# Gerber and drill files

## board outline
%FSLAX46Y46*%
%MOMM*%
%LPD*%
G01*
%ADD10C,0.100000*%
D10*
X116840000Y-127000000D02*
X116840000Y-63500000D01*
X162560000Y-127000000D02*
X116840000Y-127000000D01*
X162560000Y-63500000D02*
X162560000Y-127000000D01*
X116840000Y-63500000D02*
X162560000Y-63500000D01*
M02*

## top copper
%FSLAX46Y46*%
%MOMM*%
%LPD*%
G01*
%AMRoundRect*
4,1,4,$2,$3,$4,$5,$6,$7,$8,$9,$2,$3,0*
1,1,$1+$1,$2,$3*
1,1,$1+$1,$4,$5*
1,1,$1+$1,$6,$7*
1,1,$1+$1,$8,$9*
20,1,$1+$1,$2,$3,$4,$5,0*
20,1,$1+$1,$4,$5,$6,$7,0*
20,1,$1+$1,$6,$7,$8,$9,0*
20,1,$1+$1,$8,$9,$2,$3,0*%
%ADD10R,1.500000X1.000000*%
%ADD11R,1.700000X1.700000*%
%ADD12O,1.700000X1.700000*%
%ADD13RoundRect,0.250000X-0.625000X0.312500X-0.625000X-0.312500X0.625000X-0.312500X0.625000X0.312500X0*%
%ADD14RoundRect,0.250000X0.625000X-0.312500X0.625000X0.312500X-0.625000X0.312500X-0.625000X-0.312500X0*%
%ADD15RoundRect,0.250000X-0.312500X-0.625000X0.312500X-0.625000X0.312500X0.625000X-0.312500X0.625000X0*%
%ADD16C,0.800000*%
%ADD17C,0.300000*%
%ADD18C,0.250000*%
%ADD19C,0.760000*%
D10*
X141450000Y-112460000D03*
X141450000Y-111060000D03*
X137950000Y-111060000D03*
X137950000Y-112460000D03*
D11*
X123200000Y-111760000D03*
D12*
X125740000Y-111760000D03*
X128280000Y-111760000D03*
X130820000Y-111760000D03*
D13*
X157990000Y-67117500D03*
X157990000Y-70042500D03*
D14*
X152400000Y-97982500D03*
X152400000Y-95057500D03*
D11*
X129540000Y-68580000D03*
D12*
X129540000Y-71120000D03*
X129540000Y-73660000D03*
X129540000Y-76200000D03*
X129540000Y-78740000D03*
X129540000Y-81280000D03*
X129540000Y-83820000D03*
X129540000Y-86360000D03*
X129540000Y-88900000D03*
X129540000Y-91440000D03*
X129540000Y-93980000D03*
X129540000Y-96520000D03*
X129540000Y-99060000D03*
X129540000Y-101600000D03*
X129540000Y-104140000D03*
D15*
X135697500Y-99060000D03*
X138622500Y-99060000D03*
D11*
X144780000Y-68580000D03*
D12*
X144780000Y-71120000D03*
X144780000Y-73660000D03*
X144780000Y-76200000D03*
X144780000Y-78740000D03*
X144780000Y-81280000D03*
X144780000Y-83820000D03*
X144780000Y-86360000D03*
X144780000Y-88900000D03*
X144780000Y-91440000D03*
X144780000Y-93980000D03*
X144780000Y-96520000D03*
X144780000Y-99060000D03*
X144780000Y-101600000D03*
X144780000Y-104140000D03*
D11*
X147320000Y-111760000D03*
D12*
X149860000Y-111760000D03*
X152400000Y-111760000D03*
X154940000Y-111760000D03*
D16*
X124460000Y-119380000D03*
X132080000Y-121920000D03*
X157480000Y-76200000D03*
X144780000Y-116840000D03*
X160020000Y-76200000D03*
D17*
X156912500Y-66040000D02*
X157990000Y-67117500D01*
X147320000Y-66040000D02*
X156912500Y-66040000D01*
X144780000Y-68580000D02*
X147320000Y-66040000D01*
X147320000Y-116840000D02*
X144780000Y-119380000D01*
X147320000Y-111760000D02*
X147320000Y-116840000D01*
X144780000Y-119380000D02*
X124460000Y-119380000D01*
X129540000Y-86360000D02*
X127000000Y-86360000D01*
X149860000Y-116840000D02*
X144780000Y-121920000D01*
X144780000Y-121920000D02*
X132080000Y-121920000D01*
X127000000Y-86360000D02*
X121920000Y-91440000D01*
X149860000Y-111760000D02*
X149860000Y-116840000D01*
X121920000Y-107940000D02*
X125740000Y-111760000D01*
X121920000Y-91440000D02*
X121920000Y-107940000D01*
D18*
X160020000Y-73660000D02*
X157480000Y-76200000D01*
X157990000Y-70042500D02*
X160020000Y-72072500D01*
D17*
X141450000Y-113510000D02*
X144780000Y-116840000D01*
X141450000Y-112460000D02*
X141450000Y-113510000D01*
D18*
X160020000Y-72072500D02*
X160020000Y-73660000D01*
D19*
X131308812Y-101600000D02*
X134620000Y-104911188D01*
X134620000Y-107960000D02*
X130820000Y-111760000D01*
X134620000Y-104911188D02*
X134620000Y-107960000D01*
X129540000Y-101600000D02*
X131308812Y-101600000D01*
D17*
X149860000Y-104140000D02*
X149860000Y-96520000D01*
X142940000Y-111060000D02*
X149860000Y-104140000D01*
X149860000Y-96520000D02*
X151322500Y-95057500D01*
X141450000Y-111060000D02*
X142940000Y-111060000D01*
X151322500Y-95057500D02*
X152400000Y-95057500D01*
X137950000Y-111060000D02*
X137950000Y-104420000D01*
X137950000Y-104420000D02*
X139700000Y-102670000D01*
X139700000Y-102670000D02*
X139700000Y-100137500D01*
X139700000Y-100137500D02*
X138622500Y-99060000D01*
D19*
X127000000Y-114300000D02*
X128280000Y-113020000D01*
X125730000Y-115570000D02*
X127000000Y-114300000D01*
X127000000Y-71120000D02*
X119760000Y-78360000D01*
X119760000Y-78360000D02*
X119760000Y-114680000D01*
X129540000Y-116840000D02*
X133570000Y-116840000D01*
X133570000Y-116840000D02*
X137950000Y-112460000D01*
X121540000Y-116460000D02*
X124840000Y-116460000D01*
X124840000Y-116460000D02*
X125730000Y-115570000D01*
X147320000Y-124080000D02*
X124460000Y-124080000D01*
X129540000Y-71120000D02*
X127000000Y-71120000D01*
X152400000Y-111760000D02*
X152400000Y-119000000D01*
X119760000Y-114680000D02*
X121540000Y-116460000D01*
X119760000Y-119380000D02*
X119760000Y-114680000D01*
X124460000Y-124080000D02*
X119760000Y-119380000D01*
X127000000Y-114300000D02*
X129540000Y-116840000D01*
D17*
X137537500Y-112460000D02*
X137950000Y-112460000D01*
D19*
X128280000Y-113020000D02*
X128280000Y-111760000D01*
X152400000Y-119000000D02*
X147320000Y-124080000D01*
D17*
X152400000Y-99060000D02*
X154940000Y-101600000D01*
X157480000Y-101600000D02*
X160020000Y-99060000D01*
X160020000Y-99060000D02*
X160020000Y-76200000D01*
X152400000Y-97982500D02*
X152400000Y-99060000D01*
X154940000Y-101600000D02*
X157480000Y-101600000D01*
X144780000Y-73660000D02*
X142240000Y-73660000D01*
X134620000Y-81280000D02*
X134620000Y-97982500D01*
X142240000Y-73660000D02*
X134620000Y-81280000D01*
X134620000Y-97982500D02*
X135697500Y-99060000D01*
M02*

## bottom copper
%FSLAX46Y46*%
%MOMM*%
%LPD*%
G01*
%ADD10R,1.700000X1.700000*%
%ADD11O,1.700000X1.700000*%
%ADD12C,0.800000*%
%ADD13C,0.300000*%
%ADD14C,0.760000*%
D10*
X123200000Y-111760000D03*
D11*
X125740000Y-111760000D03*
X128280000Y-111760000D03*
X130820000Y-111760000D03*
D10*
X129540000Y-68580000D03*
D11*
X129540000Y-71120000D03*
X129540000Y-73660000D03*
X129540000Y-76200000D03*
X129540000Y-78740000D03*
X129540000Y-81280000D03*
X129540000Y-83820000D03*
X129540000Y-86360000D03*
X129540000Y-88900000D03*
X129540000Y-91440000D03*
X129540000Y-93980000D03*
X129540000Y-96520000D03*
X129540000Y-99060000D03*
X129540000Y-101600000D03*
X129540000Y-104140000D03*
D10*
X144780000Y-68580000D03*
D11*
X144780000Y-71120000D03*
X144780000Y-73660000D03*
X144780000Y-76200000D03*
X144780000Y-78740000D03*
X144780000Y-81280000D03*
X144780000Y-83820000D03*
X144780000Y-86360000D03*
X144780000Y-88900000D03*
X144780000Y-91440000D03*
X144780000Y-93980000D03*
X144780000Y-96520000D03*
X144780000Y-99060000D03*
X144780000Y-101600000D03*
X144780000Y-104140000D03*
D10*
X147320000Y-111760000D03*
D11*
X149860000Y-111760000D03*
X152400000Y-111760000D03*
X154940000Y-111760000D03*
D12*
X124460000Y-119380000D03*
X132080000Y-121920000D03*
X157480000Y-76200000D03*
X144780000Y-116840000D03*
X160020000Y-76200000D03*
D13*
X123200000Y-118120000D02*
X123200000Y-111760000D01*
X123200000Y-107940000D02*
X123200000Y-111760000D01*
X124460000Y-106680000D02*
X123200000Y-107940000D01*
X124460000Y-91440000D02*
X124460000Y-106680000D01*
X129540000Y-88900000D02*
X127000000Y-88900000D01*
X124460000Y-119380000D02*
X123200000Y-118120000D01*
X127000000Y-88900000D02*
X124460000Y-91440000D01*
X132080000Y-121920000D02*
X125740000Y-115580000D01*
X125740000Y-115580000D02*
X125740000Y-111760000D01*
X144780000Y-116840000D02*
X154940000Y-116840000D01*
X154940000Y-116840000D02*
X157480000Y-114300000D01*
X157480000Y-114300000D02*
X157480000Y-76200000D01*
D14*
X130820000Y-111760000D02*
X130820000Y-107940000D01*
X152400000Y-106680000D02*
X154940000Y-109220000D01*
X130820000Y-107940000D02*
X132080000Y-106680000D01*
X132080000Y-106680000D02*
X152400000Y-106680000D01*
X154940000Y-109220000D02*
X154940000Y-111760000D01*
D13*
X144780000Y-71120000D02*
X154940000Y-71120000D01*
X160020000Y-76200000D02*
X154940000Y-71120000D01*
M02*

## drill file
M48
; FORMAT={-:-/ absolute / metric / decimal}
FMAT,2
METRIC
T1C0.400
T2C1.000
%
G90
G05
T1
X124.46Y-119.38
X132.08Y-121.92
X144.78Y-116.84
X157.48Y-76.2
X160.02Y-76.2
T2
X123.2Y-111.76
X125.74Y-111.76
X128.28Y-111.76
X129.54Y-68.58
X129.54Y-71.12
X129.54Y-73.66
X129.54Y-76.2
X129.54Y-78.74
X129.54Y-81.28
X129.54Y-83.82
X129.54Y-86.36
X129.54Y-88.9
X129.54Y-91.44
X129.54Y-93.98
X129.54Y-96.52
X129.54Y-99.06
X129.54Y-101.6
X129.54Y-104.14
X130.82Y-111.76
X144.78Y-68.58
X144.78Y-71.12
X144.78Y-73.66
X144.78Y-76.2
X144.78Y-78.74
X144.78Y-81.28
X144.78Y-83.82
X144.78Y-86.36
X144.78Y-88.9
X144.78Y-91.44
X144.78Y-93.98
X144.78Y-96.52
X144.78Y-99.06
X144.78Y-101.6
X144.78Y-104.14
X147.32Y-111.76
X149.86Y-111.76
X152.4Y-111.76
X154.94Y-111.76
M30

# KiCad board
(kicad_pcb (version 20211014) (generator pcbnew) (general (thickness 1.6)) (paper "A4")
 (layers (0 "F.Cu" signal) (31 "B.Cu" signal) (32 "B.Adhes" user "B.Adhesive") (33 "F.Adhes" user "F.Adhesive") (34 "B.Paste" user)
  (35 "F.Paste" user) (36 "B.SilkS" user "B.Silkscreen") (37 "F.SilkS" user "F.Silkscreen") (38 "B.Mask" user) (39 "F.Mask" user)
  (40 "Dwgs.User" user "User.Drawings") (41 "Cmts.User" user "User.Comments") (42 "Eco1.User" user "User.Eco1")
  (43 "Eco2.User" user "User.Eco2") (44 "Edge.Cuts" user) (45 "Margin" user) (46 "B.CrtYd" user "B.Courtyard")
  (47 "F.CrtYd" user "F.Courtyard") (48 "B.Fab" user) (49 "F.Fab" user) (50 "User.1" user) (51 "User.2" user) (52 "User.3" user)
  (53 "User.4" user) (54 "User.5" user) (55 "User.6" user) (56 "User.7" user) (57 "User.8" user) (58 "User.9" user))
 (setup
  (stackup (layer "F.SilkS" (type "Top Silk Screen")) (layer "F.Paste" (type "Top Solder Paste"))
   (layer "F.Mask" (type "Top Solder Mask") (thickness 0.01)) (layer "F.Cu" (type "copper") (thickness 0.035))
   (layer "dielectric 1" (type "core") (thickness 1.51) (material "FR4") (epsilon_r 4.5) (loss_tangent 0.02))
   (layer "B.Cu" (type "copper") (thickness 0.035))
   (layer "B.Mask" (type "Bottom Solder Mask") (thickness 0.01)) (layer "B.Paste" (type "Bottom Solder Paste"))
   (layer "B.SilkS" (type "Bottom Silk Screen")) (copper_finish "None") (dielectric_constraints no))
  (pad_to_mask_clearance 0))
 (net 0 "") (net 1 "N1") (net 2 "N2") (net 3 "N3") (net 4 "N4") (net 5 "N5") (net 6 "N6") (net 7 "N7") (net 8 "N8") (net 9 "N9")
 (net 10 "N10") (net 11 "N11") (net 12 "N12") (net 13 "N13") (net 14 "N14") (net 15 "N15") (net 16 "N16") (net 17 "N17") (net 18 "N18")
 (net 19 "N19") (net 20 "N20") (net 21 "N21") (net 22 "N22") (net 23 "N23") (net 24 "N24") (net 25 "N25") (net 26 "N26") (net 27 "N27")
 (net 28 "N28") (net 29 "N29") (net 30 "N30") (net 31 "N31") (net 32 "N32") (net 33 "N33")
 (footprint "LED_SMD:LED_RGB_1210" (layer "F.Cu") (at 139.7 111.76 180)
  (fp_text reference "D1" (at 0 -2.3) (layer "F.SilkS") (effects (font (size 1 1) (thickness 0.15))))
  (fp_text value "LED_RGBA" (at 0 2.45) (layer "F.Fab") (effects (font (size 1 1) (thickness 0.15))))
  (pad "1" smd rect (at -1.75 -0.7) (size 1.5 1) (layers "F.Cu" "F.Paste" "F.Mask") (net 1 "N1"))
  (pad "2" smd rect (at -1.75 0.7) (size 1.5 1) (layers "F.Cu" "F.Paste" "F.Mask") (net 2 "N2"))
  (pad "3" smd rect (at 1.75 0.7) (size 1.5 1) (layers "F.Cu" "F.Paste" "F.Mask") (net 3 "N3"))
  (pad "4" smd rect (at 1.75 -0.7) (size 1.5 1) (layers "F.Cu" "F.Paste" "F.Mask") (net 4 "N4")))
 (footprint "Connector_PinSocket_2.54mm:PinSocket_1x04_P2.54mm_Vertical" (layer "F.Cu") (at 123.2 111.76 90)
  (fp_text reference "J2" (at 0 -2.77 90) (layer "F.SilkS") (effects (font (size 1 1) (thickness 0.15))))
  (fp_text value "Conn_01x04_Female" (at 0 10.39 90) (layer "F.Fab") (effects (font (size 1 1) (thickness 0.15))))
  (pad "1" thru_hole rect (at 0 0 90) (size 1.7 1.7) (drill 1) (layers *.Cu *.Mask) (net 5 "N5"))
  (pad "2" thru_hole oval (at 0 2.54 90) (size 1.7 1.7) (drill 1) (layers *.Cu *.Mask) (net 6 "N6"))
  (pad "3" thru_hole oval (at 0 5.08 90) (size 1.7 1.7) (drill 1) (layers *.Cu *.Mask) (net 4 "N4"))
  (pad "4" thru_hole oval (at 0 7.62 90) (size 1.7 1.7) (drill 1) (layers *.Cu *.Mask) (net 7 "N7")))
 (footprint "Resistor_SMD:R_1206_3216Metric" (layer "F.Cu") (at 157.99 68.58 -90)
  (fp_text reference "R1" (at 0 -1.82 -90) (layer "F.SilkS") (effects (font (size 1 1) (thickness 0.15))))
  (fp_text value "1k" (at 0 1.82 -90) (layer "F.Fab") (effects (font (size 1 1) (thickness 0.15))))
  (pad "1" smd roundrect (at -1.4625 0 270) (size 1.125 1.75) (layers "F.Cu" "F.Paste" "F.Mask") (roundrect_rratio 0.222222) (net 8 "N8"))
  (pad "2" smd roundrect (at 1.4625 0 270) (size 1.125 1.75) (layers "F.Cu" "F.Paste" "F.Mask") (roundrect_rratio 0.222222) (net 1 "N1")))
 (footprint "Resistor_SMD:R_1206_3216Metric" (layer "F.Cu") (at 152.4 96.52 90)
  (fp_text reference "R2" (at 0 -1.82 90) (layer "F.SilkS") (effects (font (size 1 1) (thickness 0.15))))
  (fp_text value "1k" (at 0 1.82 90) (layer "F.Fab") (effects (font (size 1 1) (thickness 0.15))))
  (pad "1" smd roundrect (at -1.4625 0 90) (size 1.125 1.75) (layers "F.Cu" "F.Paste" "F.Mask") (roundrect_rratio 0.222222) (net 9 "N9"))
  (pad "2" smd roundrect (at 1.4625 0 90) (size 1.125 1.75) (layers "F.Cu" "F.Paste" "F.Mask") (roundrect_rratio 0.222222) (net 2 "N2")))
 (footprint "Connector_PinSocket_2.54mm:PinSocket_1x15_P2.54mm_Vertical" (layer "F.Cu") (at 129.54 68.58)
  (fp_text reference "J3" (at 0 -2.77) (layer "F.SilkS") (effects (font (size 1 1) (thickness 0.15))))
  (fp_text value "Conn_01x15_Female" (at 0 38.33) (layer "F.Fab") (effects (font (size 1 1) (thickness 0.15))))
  (pad "1" thru_hole rect (at 0 0) (size 1.7 1.7) (drill 1) (layers *.Cu *.Mask) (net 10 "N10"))
  (pad "2" thru_hole oval (at 0 2.54) (size 1.7 1.7) (drill 1) (layers *.Cu *.Mask) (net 4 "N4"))
  (pad "3" thru_hole oval (at 0 5.08) (size 1.7 1.7) (drill 1) (layers *.Cu *.Mask) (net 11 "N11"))
  (pad "4" thru_hole oval (at 0 7.62) (size 1.7 1.7) (drill 1) (layers *.Cu *.Mask) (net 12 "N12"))
  (pad "5" thru_hole oval (at 0 10.16) (size 1.7 1.7) (drill 1) (layers *.Cu *.Mask) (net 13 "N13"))
  (pad "6" thru_hole oval (at 0 12.7) (size 1.7 1.7) (drill 1) (layers *.Cu *.Mask) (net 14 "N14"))
  (pad "7" thru_hole oval (at 0 15.24) (size 1.7 1.7) (drill 1) (layers *.Cu *.Mask) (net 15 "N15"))
  (pad "8" thru_hole oval (at 0 17.78) (size 1.7 1.7) (drill 1) (layers *.Cu *.Mask) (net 6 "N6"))
  (pad "9" thru_hole oval (at 0 20.32) (size 1.7 1.7) (drill 1) (layers *.Cu *.Mask) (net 5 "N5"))
  (pad "10" thru_hole oval (at 0 22.86) (size 1.7 1.7) (drill 1) (layers *.Cu *.Mask) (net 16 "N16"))
  (pad "11" thru_hole oval (at 0 25.4) (size 1.7 1.7) (drill 1) (layers *.Cu *.Mask) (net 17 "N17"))
  (pad "12" thru_hole oval (at 0 27.94) (size 1.7 1.7) (drill 1) (layers *.Cu *.Mask) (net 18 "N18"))
  (pad "13" thru_hole oval (at 0 30.48) (size 1.7 1.7) (drill 1) (layers *.Cu *.Mask) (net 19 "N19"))
  (pad "14" thru_hole oval (at 0 33.02) (size 1.7 1.7) (drill 1) (layers *.Cu *.Mask) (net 7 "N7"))
  (pad "15" thru_hole oval (at 0 35.56) (size 1.7 1.7) (drill 1) (layers *.Cu *.Mask) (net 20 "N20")))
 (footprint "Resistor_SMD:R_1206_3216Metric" (layer "F.Cu") (at 137.16 99.06)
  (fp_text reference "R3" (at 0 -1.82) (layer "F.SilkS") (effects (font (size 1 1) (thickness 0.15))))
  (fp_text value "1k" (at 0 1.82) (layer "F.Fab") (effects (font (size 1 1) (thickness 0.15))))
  (pad "1" smd roundrect (at -1.4625 0) (size 1.125 1.75) (layers "F.Cu" "F.Paste" "F.Mask") (roundrect_rratio 0.222222) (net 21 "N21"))
  (pad "2" smd roundrect (at 1.4625 0) (size 1.125 1.75) (layers "F.Cu" "F.Paste" "F.Mask") (roundrect_rratio 0.222222) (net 3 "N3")))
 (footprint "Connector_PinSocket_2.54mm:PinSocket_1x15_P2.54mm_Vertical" (layer "F.Cu") (at 144.78 68.58)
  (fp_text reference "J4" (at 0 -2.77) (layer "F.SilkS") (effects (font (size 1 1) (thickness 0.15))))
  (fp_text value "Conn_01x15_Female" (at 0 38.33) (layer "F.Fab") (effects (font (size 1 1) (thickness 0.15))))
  (pad "1" thru_hole rect (at 0 0) (size 1.7 1.7) (drill 1) (layers *.Cu *.Mask) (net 8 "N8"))
  (pad "2" thru_hole oval (at 0 2.54) (size 1.7 1.7) (drill 1) (layers *.Cu *.Mask) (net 9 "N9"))
  (pad "3" thru_hole oval (at 0 5.08) (size 1.7 1.7) (drill 1) (layers *.Cu *.Mask) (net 21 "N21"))
  (pad "4" thru_hole oval (at 0 7.62) (size 1.7 1.7) (drill 1) (layers *.Cu *.Mask) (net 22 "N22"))
  (pad "5" thru_hole oval (at 0 10.16) (size 1.7 1.7) (drill 1) (layers *.Cu *.Mask) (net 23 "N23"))
  (pad "6" thru_hole oval (at 0 12.7) (size 1.7 1.7) (drill 1) (layers *.Cu *.Mask) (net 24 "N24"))
  (pad "7" thru_hole oval (at 0 15.24) (size 1.7 1.7) (drill 1) (layers *.Cu *.Mask) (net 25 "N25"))
  (pad "8" thru_hole oval (at 0 17.78) (size 1.7 1.7) (drill 1) (layers *.Cu *.Mask) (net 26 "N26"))
  (pad "9" thru_hole oval (at 0 20.32) (size 1.7 1.7) (drill 1) (layers *.Cu *.Mask) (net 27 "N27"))
  (pad "10" thru_hole oval (at 0 22.86) (size 1.7 1.7) (drill 1) (layers *.Cu *.Mask) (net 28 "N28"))
  (pad "11" thru_hole oval (at 0 25.4) (size 1.7 1.7) (drill 1) (layers *.Cu *.Mask) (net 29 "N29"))
  (pad "12" thru_hole oval (at 0 27.94) (size 1.7 1.7) (drill 1) (layers *.Cu *.Mask) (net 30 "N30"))
  (pad "13" thru_hole oval (at 0 30.48) (size 1.7 1.7) (drill 1) (layers *.Cu *.Mask) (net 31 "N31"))
  (pad "14" thru_hole oval (at 0 33.02) (size 1.7 1.7) (drill 1) (layers *.Cu *.Mask) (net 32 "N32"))
  (pad "15" thru_hole oval (at 0 35.56) (size 1.7 1.7) (drill 1) (layers *.Cu *.Mask) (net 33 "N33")))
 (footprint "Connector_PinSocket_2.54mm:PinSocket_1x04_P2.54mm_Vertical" (layer "F.Cu") (at 147.32 111.76 90)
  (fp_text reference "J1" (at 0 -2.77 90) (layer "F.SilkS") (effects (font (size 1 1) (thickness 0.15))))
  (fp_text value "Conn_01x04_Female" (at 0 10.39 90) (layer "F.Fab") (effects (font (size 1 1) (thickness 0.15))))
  (pad "1" thru_hole rect (at 0 0 90) (size 1.7 1.7) (drill 1) (layers *.Cu *.Mask) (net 5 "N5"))
  (pad "2" thru_hole oval (at 0 2.54 90) (size 1.7 1.7) (drill 1) (layers *.Cu *.Mask) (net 6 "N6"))
  (pad "3" thru_hole oval (at 0 5.08 90) (size 1.7 1.7) (drill 1) (layers *.Cu *.Mask) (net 4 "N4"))
  (pad "4" thru_hole oval (at 0 7.62 90) (size 1.7 1.7) (drill 1) (layers *.Cu *.Mask) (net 7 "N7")))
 (gr_line (start 116.84 127) (end 116.84 63.5) (layer "Edge.Cuts") (width 0.1))
 (gr_line (start 162.56 127) (end 116.84 127) (layer "Edge.Cuts") (width 0.1))
 (gr_line (start 162.56 63.5) (end 162.56 127) (layer "Edge.Cuts") (width 0.1))
 (gr_line (start 116.84 63.5) (end 162.56 63.5) (layer "Edge.Cuts") (width 0.1))
 (segment (start 156.9125 66.04) (end 157.99 67.1175) (width 0.3) (layer "F.Cu") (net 8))
 (segment (start 147.32 66.04) (end 156.9125 66.04) (width 0.3) (layer "F.Cu") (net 8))
 (segment (start 144.78 68.58) (end 147.32 66.04) (width 0.3) (layer "F.Cu") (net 8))
 (segment (start 147.32 116.84) (end 144.78 119.38) (width 0.3) (layer "F.Cu") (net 5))
 (segment (start 147.32 111.76) (end 147.32 116.84) (width 0.3) (layer "F.Cu") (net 5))
 (segment (start 144.78 119.38) (end 124.46 119.38) (width 0.3) (layer "F.Cu") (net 5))
 (via (at 124.46 119.38) (size 0.8) (drill 0.4) (layers "F.Cu" "B.Cu") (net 5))
 (segment (start 123.2 118.12) (end 123.2 111.76) (width 0.3) (layer "B.Cu") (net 5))
 (segment (start 123.2 107.94) (end 123.2 111.76) (width 0.3) (layer "B.Cu") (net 5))
 (segment (start 124.46 106.68) (end 123.2 107.94) (width 0.3) (layer "B.Cu") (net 5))
 (segment (start 124.46 91.44) (end 124.46 106.68) (width 0.3) (layer "B.Cu") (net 5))
 (segment (start 129.54 88.9) (end 127 88.9) (width 0.3) (layer "B.Cu") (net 5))
 (segment (start 124.46 119.38) (end 123.2 118.12) (width 0.3) (layer "B.Cu") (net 5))
 (segment (start 127 88.9) (end 124.46 91.44) (width 0.3) (layer "B.Cu") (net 5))
 (segment (start 129.54 86.36) (end 127 86.36) (width 0.3) (layer "F.Cu") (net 6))
 (segment (start 149.86 116.84) (end 144.78 121.92) (width 0.3) (layer "F.Cu") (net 6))
 (segment (start 144.78 121.92) (end 132.08 121.92) (width 0.3) (layer "F.Cu") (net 6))
 (segment (start 127 86.36) (end 121.92 91.44) (width 0.3) (layer "F.Cu") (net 6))
 (segment (start 149.86 111.76) (end 149.86 116.84) (width 0.3) (layer "F.Cu") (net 6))
 (segment (start 121.92 107.94) (end 125.74 111.76) (width 0.3) (layer "F.Cu") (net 6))
 (segment (start 121.92 91.44) (end 121.92 107.94) (width 0.3) (layer "F.Cu") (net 6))
 (via (at 132.08 121.92) (size 0.8) (drill 0.4) (layers "F.Cu" "B.Cu") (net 6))
 (segment (start 132.08 121.92) (end 125.74 115.58) (width 0.3) (layer "B.Cu") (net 6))
 (segment (start 125.74 115.58) (end 125.74 111.76) (width 0.3) (layer "B.Cu") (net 6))
 (segment (start 160.02 73.66) (end 157.48 76.2) (width 0.25) (layer "F.Cu") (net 1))
 (segment (start 157.99 70.0425) (end 160.02 72.0725) (width 0.25) (layer "F.Cu") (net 1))
 (segment (start 141.45 113.51) (end 144.78 116.84) (width 0.3) (layer "F.Cu") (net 1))
 (segment (start 141.45 112.46) (end 141.45 113.51) (width 0.3) (layer "F.Cu") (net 1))
 (segment (start 160.02 72.0725) (end 160.02 73.66) (width 0.25) (layer "F.Cu") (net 1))
 (via (at 157.48 76.2) (size 0.8) (drill 0.4) (layers "F.Cu" "B.Cu") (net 1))
 (via (at 144.78 116.84) (size 0.8) (drill 0.4) (layers "F.Cu" "B.Cu") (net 1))
 (segment (start 144.78 116.84) (end 154.94 116.84) (width 0.3) (layer "B.Cu") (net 1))
 (segment (start 154.94 116.84) (end 157.48 114.3) (width 0.3) (layer "B.Cu") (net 1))
 (segment (start 157.48 114.3) (end 157.48 76.2) (width 0.3) (layer "B.Cu") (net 1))
 (segment (start 131.308812 101.6) (end 134.62 104.911188) (width 0.76) (layer "F.Cu") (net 7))
 (segment (start 134.62 107.96) (end 130.82 111.76) (width 0.76) (layer "F.Cu") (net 7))
 (segment (start 134.62 104.911188) (end 134.62 107.96) (width 0.76) (layer "F.Cu") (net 7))
 (segment (start 129.54 101.6) (end 131.308812 101.6) (width 0.76) (layer "F.Cu") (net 7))
 (segment (start 130.82 111.76) (end 130.82 107.94) (width 0.76) (layer "B.Cu") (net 7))
 (segment (start 152.4 106.68) (end 154.94 109.22) (width 0.76) (layer "B.Cu") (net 7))
 (segment (start 130.82 107.94) (end 132.08 106.68) (width 0.76) (layer "B.Cu") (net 7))
 (segment (start 132.08 106.68) (end 152.4 106.68) (width 0.76) (layer "B.Cu") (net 7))
 (segment (start 154.94 109.22) (end 154.94 111.76) (width 0.76) (layer "B.Cu") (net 7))
 (segment (start 149.86 104.14) (end 149.86 96.52) (width 0.3) (layer "F.Cu") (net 2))
 (segment (start 142.94 111.06) (end 149.86 104.14) (width 0.3) (layer "F.Cu") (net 2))
 (segment (start 149.86 96.52) (end 151.3225 95.0575) (width 0.3) (layer "F.Cu") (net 2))
 (segment (start 141.45 111.06) (end 142.94 111.06) (width 0.3) (layer "F.Cu") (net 2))
 (segment (start 151.3225 95.0575) (end 152.4 95.0575) (width 0.3) (layer "F.Cu") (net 2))
 (segment (start 137.95 111.06) (end 137.95 104.42) (width 0.3) (layer "F.Cu") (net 3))
 (segment (start 137.95 104.42) (end 139.7 102.67) (width 0.3) (layer "F.Cu") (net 3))
 (segment (start 139.7 102.67) (end 139.7 100.1375) (width 0.3) (layer "F.Cu") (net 3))
 (segment (start 139.7 100.1375) (end 138.6225 99.06) (width 0.3) (layer "F.Cu") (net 3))
 (segment (start 127 114.3) (end 128.28 113.02) (width 0.76) (layer "F.Cu") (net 4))
 (segment (start 125.73 115.57) (end 127 114.3) (width 0.76) (layer "F.Cu") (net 4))
 (segment (start 127 71.12) (end 119.76 78.36) (width 0.76) (layer "F.Cu") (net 4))
 (segment (start 119.76 78.36) (end 119.76 114.68) (width 0.76) (layer "F.Cu") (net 4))
 (segment (start 129.54 116.84) (end 133.57 116.84) (width 0.76) (layer "F.Cu") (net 4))
 (segment (start 133.57 116.84) (end 137.95 112.46) (width 0.76) (layer "F.Cu") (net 4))
 (segment (start 121.54 116.46) (end 124.84 116.46) (width 0.76) (layer "F.Cu") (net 4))
 (segment (start 124.84 116.46) (end 125.73 115.57) (width 0.76) (layer "F.Cu") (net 4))
 (segment (start 147.32 124.08) (end 124.46 124.08) (width 0.76) (layer "F.Cu") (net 4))
 (segment (start 129.54 71.12) (end 127 71.12) (width 0.76) (layer "F.Cu") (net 4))
 (segment (start 152.4 111.76) (end 152.4 119) (width 0.76) (layer "F.Cu") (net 4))
 (segment (start 119.76 114.68) (end 121.54 116.46) (width 0.76) (layer "F.Cu") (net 4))
 (segment (start 119.76 119.38) (end 119.76 114.68) (width 0.76) (layer "F.Cu") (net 4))
 (segment (start 124.46 124.08) (end 119.76 119.38) (width 0.76) (layer "F.Cu") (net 4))
 (segment (start 127 114.3) (end 129.54 116.84) (width 0.76) (layer "F.Cu") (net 4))
 (segment (start 137.5375 112.46) (end 137.95 112.46) (width 0.3) (layer "F.Cu") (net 4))
 (segment (start 128.28 113.02) (end 128.28 111.76) (width 0.76) (layer "F.Cu") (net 4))
 (segment (start 152.4 119) (end 147.32 124.08) (width 0.76) (layer "F.Cu") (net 4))
 (segment (start 152.4 99.06) (end 154.94 101.6) (width 0.3) (layer "F.Cu") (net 9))
 (segment (start 157.48 101.6) (end 160.02 99.06) (width 0.3) (layer "F.Cu") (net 9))
 (segment (start 160.02 99.06) (end 160.02 76.2) (width 0.3) (layer "F.Cu") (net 9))
 (segment (start 152.4 97.9825) (end 152.4 99.06) (width 0.3) (layer "F.Cu") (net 9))
 (segment (start 154.94 101.6) (end 157.48 101.6) (width 0.3) (layer "F.Cu") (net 9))
 (via (at 160.02 76.2) (size 0.8) (drill 0.4) (layers "F.Cu" "B.Cu") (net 9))
 (segment (start 144.78 71.12) (end 154.94 71.12) (width 0.3) (layer "B.Cu") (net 9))
 (segment (start 160.02 76.2) (end 154.94 71.12) (width 0.3) (layer "B.Cu") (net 9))
 (segment (start 144.78 73.66) (end 142.24 73.66) (width 0.3) (layer "F.Cu") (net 21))
 (segment (start 134.62 81.28) (end 134.62 97.9825) (width 0.3) (layer "F.Cu") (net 21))
 (segment (start 142.24 73.66) (end 134.62 81.28) (width 0.3) (layer "F.Cu") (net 21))
 (segment (start 134.62 97.9825) (end 135.6975 99.06) (width 0.3) (layer "F.Cu") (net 21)))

